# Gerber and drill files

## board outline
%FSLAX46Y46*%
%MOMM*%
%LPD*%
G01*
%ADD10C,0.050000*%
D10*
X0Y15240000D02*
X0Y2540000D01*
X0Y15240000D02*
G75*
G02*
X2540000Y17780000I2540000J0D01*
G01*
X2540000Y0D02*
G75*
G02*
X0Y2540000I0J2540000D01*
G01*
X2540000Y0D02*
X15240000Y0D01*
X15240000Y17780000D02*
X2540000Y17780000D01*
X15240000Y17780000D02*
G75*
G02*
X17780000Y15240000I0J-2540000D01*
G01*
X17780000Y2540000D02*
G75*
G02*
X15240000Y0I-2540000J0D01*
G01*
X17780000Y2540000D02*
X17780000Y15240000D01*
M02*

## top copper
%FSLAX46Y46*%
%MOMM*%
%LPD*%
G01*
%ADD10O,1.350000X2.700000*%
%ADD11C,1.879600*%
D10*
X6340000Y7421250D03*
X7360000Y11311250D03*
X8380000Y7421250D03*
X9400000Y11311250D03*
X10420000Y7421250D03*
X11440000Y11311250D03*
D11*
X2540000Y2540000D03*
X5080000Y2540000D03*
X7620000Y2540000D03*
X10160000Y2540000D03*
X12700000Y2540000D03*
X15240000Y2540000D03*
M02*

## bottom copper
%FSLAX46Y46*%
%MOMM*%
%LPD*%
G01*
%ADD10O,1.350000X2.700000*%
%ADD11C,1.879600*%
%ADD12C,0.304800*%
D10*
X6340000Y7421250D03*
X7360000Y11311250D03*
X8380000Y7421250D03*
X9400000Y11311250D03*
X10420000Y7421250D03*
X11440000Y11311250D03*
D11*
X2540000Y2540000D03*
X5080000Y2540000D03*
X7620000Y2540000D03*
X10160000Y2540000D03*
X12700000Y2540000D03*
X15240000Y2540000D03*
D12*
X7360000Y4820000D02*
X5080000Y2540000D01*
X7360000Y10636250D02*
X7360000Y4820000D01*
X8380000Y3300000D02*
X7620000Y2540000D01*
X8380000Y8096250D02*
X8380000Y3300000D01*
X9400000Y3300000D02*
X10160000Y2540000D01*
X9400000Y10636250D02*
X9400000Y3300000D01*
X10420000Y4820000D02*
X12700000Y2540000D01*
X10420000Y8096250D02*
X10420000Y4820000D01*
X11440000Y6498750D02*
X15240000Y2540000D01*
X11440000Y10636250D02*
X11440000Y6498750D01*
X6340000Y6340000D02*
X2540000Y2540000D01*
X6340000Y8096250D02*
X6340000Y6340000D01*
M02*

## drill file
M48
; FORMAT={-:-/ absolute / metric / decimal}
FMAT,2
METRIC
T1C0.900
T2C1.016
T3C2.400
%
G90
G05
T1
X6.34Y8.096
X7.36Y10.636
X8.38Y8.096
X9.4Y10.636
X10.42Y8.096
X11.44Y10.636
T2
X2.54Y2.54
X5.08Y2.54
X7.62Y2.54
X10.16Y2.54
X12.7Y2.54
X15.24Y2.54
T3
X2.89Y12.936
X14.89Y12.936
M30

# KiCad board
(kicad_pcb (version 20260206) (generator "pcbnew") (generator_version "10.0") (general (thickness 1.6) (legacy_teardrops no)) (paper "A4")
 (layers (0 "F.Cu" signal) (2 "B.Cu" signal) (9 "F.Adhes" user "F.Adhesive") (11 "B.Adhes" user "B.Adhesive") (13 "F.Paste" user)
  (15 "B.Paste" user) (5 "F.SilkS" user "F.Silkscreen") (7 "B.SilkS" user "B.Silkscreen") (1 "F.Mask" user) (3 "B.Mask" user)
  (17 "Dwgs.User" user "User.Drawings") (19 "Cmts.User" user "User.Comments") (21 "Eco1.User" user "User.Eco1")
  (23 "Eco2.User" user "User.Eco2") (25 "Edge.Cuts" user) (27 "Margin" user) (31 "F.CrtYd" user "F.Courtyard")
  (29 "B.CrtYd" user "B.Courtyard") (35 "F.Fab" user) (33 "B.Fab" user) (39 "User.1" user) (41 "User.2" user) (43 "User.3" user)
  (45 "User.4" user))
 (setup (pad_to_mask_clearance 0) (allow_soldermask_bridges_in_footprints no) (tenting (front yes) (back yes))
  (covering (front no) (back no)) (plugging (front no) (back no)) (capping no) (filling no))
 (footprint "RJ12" (layer "F.Cu") (at 8.89 -10.63625 180)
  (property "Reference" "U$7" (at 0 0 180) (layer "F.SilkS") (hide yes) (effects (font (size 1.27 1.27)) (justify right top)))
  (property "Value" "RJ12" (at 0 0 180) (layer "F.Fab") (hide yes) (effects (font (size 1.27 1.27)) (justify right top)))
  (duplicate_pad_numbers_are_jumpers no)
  (pad "" np_thru_hole circle (at -6 2.3 180) (size 2.4 2.4) (drill 2.4) (layers "*.Cu" "*.Mask"))
  (pad "" np_thru_hole circle (at 6 2.3 180) (size 2.4 2.4) (drill 2.4) (layers "*.Cu" "*.Mask"))
  (pad "1" thru_hole oval (at 2.55 -2.54 270) (size 2.7 1.35) (drill 0.9 (offset 0.675 0)) (layers "*.Cu" "*.Mask")
   (remove_unused_layers no) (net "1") (solder_mask_margin 0.0762) (thermal_bridge_angle 0))
  (pad "2" thru_hole oval (at 1.53 0 90) (size 2.7 1.35) (drill 0.9 (offset 0.675 0)) (layers "*.Cu" "*.Mask") (remove_unused_layers no)
   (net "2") (solder_mask_margin 0.0762) (thermal_bridge_angle 0))
  (pad "3" thru_hole oval (at 0.51 -2.54 270) (size 2.7 1.35) (drill 0.9 (offset 0.675 0)) (layers "*.Cu" "*.Mask")
   (remove_unused_layers no) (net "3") (solder_mask_margin 0.0762) (thermal_bridge_angle 0))
  (pad "4" thru_hole oval (at -0.51 0 90) (size 2.7 1.35) (drill 0.9 (offset 0.675 0)) (layers "*.Cu" "*.Mask") (remove_unused_layers no)
   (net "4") (solder_mask_margin 0.0762) (thermal_bridge_angle 0))
  (pad "5" thru_hole oval (at -1.53 -2.54 270) (size 2.7 1.35) (drill 0.9 (offset 0.675 0)) (layers "*.Cu" "*.Mask")
   (remove_unused_layers no) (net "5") (solder_mask_margin 0.0762) (thermal_bridge_angle 0))
  (pad "6" thru_hole oval (at -2.55 0 90) (size 2.7 1.35) (drill 0.9 (offset 0.675 0)) (layers "*.Cu" "*.Mask") (remove_unused_layers no)
   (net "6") (solder_mask_margin 0.0762) (thermal_bridge_angle 0)))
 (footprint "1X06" (layer "F.Cu") (at 2.54 -2.54)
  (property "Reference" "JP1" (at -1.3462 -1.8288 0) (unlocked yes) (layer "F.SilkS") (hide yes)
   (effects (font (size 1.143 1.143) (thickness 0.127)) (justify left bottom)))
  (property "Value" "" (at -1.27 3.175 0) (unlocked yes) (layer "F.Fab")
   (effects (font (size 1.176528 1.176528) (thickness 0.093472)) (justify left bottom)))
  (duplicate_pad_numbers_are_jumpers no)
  (pad "1" thru_hole circle (at 0 0 90) (size 1.8796 1.8796) (drill 1.016) (layers "*.Cu" "*.Mask") (remove_unused_layers no) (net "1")
   (solder_mask_margin 0.0762) (thermal_bridge_angle 0))
  (pad "2" thru_hole circle (at 2.54 0 90) (size 1.8796 1.8796) (drill 1.016) (layers "*.Cu" "*.Mask") (remove_unused_layers no) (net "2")
   (solder_mask_margin 0.0762) (thermal_bridge_angle 0))
  (pad "3" thru_hole circle (at 5.08 0 90) (size 1.8796 1.8796) (drill 1.016) (layers "*.Cu" "*.Mask") (remove_unused_layers no) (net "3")
   (solder_mask_margin 0.0762) (thermal_bridge_angle 0))
  (pad "4" thru_hole circle (at 7.62 0 90) (size 1.8796 1.8796) (drill 1.016) (layers "*.Cu" "*.Mask") (remove_unused_layers no) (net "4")
   (solder_mask_margin 0.0762) (thermal_bridge_angle 0))
  (pad "5" thru_hole circle (at 10.16 0 90) (size 1.8796 1.8796) (drill 1.016) (layers "*.Cu" "*.Mask") (remove_unused_layers no) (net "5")
   (solder_mask_margin 0.0762) (thermal_bridge_angle 0))
  (pad "6" thru_hole circle (at 12.7 0 90) (size 1.8796 1.8796) (drill 1.016) (layers "*.Cu" "*.Mask") (remove_unused_layers no) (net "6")
   (solder_mask_margin 0.0762) (thermal_bridge_angle 0)))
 (gr_line (start 0 -15.24) (end 0 -2.54) (stroke (width 0.05) (type solid)) (layer "Edge.Cuts"))
 (gr_arc (start 0 -15.24) (mid 0.743949 -17.036051) (end 2.54 -17.78) (stroke (width 0.05) (type solid)) (layer "Edge.Cuts"))
 (gr_arc (start 2.54 0) (mid 0.743949 -0.743949) (end 0 -2.54) (stroke (width 0.05) (type solid)) (layer "Edge.Cuts"))
 (gr_line (start 2.54 0) (end 15.24 0) (stroke (width 0.05) (type solid)) (layer "Edge.Cuts"))
 (gr_line (start 15.24 -17.78) (end 2.54 -17.78) (stroke (width 0.05) (type solid)) (layer "Edge.Cuts"))
 (gr_arc (start 15.24 -17.78) (mid 17.036051 -17.036051) (end 17.78 -15.24) (stroke (width 0.05) (type solid)) (layer "Edge.Cuts"))
 (gr_arc (start 17.78 -2.54) (mid 17.036051 -0.743949) (end 15.24 0) (stroke (width 0.05) (type solid)) (layer "Edge.Cuts"))
 (gr_line (start 17.78 -2.54) (end 17.78 -15.24) (stroke (width 0.05) (type solid)) (layer "Edge.Cuts"))
 (segment (start 7.36 -4.82) (end 5.08 -2.54) (width 0.3048) (layer "B.Cu") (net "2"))
 (segment (start 7.36 -10.63625) (end 7.36 -4.82) (width 0.3048) (layer "B.Cu") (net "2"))
 (segment (start 8.38 -3.3) (end 7.62 -2.54) (width 0.3048) (layer "B.Cu") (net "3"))
 (segment (start 8.38 -8.09625) (end 8.38 -3.3) (width 0.3048) (layer "B.Cu") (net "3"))
 (segment (start 9.4 -3.3) (end 10.16 -2.54) (width 0.3048) (layer "B.Cu") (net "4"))
 (segment (start 9.4 -10.63625) (end 9.4 -3.3) (width 0.3048) (layer "B.Cu") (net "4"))
 (segment (start 10.42 -4.82) (end 12.7 -2.54) (width 0.3048) (layer "B.Cu") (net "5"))
 (segment (start 10.42 -8.09625) (end 10.42 -4.82) (width 0.3048) (layer "B.Cu") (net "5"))
 (segment (start 11.44 -6.49875) (end 15.24 -2.54) (width 0.3048) (layer "B.Cu") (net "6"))
 (segment (start 11.44 -10.63625) (end 11.44 -6.49875) (width 0.3048) (layer "B.Cu") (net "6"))
 (segment (start 6.34 -6.34) (end 2.54 -2.54) (width 0.3048) (layer "B.Cu") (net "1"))
 (segment (start 6.34 -8.09625) (end 6.34 -6.34) (width 0.3048) (layer "B.Cu") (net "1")))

